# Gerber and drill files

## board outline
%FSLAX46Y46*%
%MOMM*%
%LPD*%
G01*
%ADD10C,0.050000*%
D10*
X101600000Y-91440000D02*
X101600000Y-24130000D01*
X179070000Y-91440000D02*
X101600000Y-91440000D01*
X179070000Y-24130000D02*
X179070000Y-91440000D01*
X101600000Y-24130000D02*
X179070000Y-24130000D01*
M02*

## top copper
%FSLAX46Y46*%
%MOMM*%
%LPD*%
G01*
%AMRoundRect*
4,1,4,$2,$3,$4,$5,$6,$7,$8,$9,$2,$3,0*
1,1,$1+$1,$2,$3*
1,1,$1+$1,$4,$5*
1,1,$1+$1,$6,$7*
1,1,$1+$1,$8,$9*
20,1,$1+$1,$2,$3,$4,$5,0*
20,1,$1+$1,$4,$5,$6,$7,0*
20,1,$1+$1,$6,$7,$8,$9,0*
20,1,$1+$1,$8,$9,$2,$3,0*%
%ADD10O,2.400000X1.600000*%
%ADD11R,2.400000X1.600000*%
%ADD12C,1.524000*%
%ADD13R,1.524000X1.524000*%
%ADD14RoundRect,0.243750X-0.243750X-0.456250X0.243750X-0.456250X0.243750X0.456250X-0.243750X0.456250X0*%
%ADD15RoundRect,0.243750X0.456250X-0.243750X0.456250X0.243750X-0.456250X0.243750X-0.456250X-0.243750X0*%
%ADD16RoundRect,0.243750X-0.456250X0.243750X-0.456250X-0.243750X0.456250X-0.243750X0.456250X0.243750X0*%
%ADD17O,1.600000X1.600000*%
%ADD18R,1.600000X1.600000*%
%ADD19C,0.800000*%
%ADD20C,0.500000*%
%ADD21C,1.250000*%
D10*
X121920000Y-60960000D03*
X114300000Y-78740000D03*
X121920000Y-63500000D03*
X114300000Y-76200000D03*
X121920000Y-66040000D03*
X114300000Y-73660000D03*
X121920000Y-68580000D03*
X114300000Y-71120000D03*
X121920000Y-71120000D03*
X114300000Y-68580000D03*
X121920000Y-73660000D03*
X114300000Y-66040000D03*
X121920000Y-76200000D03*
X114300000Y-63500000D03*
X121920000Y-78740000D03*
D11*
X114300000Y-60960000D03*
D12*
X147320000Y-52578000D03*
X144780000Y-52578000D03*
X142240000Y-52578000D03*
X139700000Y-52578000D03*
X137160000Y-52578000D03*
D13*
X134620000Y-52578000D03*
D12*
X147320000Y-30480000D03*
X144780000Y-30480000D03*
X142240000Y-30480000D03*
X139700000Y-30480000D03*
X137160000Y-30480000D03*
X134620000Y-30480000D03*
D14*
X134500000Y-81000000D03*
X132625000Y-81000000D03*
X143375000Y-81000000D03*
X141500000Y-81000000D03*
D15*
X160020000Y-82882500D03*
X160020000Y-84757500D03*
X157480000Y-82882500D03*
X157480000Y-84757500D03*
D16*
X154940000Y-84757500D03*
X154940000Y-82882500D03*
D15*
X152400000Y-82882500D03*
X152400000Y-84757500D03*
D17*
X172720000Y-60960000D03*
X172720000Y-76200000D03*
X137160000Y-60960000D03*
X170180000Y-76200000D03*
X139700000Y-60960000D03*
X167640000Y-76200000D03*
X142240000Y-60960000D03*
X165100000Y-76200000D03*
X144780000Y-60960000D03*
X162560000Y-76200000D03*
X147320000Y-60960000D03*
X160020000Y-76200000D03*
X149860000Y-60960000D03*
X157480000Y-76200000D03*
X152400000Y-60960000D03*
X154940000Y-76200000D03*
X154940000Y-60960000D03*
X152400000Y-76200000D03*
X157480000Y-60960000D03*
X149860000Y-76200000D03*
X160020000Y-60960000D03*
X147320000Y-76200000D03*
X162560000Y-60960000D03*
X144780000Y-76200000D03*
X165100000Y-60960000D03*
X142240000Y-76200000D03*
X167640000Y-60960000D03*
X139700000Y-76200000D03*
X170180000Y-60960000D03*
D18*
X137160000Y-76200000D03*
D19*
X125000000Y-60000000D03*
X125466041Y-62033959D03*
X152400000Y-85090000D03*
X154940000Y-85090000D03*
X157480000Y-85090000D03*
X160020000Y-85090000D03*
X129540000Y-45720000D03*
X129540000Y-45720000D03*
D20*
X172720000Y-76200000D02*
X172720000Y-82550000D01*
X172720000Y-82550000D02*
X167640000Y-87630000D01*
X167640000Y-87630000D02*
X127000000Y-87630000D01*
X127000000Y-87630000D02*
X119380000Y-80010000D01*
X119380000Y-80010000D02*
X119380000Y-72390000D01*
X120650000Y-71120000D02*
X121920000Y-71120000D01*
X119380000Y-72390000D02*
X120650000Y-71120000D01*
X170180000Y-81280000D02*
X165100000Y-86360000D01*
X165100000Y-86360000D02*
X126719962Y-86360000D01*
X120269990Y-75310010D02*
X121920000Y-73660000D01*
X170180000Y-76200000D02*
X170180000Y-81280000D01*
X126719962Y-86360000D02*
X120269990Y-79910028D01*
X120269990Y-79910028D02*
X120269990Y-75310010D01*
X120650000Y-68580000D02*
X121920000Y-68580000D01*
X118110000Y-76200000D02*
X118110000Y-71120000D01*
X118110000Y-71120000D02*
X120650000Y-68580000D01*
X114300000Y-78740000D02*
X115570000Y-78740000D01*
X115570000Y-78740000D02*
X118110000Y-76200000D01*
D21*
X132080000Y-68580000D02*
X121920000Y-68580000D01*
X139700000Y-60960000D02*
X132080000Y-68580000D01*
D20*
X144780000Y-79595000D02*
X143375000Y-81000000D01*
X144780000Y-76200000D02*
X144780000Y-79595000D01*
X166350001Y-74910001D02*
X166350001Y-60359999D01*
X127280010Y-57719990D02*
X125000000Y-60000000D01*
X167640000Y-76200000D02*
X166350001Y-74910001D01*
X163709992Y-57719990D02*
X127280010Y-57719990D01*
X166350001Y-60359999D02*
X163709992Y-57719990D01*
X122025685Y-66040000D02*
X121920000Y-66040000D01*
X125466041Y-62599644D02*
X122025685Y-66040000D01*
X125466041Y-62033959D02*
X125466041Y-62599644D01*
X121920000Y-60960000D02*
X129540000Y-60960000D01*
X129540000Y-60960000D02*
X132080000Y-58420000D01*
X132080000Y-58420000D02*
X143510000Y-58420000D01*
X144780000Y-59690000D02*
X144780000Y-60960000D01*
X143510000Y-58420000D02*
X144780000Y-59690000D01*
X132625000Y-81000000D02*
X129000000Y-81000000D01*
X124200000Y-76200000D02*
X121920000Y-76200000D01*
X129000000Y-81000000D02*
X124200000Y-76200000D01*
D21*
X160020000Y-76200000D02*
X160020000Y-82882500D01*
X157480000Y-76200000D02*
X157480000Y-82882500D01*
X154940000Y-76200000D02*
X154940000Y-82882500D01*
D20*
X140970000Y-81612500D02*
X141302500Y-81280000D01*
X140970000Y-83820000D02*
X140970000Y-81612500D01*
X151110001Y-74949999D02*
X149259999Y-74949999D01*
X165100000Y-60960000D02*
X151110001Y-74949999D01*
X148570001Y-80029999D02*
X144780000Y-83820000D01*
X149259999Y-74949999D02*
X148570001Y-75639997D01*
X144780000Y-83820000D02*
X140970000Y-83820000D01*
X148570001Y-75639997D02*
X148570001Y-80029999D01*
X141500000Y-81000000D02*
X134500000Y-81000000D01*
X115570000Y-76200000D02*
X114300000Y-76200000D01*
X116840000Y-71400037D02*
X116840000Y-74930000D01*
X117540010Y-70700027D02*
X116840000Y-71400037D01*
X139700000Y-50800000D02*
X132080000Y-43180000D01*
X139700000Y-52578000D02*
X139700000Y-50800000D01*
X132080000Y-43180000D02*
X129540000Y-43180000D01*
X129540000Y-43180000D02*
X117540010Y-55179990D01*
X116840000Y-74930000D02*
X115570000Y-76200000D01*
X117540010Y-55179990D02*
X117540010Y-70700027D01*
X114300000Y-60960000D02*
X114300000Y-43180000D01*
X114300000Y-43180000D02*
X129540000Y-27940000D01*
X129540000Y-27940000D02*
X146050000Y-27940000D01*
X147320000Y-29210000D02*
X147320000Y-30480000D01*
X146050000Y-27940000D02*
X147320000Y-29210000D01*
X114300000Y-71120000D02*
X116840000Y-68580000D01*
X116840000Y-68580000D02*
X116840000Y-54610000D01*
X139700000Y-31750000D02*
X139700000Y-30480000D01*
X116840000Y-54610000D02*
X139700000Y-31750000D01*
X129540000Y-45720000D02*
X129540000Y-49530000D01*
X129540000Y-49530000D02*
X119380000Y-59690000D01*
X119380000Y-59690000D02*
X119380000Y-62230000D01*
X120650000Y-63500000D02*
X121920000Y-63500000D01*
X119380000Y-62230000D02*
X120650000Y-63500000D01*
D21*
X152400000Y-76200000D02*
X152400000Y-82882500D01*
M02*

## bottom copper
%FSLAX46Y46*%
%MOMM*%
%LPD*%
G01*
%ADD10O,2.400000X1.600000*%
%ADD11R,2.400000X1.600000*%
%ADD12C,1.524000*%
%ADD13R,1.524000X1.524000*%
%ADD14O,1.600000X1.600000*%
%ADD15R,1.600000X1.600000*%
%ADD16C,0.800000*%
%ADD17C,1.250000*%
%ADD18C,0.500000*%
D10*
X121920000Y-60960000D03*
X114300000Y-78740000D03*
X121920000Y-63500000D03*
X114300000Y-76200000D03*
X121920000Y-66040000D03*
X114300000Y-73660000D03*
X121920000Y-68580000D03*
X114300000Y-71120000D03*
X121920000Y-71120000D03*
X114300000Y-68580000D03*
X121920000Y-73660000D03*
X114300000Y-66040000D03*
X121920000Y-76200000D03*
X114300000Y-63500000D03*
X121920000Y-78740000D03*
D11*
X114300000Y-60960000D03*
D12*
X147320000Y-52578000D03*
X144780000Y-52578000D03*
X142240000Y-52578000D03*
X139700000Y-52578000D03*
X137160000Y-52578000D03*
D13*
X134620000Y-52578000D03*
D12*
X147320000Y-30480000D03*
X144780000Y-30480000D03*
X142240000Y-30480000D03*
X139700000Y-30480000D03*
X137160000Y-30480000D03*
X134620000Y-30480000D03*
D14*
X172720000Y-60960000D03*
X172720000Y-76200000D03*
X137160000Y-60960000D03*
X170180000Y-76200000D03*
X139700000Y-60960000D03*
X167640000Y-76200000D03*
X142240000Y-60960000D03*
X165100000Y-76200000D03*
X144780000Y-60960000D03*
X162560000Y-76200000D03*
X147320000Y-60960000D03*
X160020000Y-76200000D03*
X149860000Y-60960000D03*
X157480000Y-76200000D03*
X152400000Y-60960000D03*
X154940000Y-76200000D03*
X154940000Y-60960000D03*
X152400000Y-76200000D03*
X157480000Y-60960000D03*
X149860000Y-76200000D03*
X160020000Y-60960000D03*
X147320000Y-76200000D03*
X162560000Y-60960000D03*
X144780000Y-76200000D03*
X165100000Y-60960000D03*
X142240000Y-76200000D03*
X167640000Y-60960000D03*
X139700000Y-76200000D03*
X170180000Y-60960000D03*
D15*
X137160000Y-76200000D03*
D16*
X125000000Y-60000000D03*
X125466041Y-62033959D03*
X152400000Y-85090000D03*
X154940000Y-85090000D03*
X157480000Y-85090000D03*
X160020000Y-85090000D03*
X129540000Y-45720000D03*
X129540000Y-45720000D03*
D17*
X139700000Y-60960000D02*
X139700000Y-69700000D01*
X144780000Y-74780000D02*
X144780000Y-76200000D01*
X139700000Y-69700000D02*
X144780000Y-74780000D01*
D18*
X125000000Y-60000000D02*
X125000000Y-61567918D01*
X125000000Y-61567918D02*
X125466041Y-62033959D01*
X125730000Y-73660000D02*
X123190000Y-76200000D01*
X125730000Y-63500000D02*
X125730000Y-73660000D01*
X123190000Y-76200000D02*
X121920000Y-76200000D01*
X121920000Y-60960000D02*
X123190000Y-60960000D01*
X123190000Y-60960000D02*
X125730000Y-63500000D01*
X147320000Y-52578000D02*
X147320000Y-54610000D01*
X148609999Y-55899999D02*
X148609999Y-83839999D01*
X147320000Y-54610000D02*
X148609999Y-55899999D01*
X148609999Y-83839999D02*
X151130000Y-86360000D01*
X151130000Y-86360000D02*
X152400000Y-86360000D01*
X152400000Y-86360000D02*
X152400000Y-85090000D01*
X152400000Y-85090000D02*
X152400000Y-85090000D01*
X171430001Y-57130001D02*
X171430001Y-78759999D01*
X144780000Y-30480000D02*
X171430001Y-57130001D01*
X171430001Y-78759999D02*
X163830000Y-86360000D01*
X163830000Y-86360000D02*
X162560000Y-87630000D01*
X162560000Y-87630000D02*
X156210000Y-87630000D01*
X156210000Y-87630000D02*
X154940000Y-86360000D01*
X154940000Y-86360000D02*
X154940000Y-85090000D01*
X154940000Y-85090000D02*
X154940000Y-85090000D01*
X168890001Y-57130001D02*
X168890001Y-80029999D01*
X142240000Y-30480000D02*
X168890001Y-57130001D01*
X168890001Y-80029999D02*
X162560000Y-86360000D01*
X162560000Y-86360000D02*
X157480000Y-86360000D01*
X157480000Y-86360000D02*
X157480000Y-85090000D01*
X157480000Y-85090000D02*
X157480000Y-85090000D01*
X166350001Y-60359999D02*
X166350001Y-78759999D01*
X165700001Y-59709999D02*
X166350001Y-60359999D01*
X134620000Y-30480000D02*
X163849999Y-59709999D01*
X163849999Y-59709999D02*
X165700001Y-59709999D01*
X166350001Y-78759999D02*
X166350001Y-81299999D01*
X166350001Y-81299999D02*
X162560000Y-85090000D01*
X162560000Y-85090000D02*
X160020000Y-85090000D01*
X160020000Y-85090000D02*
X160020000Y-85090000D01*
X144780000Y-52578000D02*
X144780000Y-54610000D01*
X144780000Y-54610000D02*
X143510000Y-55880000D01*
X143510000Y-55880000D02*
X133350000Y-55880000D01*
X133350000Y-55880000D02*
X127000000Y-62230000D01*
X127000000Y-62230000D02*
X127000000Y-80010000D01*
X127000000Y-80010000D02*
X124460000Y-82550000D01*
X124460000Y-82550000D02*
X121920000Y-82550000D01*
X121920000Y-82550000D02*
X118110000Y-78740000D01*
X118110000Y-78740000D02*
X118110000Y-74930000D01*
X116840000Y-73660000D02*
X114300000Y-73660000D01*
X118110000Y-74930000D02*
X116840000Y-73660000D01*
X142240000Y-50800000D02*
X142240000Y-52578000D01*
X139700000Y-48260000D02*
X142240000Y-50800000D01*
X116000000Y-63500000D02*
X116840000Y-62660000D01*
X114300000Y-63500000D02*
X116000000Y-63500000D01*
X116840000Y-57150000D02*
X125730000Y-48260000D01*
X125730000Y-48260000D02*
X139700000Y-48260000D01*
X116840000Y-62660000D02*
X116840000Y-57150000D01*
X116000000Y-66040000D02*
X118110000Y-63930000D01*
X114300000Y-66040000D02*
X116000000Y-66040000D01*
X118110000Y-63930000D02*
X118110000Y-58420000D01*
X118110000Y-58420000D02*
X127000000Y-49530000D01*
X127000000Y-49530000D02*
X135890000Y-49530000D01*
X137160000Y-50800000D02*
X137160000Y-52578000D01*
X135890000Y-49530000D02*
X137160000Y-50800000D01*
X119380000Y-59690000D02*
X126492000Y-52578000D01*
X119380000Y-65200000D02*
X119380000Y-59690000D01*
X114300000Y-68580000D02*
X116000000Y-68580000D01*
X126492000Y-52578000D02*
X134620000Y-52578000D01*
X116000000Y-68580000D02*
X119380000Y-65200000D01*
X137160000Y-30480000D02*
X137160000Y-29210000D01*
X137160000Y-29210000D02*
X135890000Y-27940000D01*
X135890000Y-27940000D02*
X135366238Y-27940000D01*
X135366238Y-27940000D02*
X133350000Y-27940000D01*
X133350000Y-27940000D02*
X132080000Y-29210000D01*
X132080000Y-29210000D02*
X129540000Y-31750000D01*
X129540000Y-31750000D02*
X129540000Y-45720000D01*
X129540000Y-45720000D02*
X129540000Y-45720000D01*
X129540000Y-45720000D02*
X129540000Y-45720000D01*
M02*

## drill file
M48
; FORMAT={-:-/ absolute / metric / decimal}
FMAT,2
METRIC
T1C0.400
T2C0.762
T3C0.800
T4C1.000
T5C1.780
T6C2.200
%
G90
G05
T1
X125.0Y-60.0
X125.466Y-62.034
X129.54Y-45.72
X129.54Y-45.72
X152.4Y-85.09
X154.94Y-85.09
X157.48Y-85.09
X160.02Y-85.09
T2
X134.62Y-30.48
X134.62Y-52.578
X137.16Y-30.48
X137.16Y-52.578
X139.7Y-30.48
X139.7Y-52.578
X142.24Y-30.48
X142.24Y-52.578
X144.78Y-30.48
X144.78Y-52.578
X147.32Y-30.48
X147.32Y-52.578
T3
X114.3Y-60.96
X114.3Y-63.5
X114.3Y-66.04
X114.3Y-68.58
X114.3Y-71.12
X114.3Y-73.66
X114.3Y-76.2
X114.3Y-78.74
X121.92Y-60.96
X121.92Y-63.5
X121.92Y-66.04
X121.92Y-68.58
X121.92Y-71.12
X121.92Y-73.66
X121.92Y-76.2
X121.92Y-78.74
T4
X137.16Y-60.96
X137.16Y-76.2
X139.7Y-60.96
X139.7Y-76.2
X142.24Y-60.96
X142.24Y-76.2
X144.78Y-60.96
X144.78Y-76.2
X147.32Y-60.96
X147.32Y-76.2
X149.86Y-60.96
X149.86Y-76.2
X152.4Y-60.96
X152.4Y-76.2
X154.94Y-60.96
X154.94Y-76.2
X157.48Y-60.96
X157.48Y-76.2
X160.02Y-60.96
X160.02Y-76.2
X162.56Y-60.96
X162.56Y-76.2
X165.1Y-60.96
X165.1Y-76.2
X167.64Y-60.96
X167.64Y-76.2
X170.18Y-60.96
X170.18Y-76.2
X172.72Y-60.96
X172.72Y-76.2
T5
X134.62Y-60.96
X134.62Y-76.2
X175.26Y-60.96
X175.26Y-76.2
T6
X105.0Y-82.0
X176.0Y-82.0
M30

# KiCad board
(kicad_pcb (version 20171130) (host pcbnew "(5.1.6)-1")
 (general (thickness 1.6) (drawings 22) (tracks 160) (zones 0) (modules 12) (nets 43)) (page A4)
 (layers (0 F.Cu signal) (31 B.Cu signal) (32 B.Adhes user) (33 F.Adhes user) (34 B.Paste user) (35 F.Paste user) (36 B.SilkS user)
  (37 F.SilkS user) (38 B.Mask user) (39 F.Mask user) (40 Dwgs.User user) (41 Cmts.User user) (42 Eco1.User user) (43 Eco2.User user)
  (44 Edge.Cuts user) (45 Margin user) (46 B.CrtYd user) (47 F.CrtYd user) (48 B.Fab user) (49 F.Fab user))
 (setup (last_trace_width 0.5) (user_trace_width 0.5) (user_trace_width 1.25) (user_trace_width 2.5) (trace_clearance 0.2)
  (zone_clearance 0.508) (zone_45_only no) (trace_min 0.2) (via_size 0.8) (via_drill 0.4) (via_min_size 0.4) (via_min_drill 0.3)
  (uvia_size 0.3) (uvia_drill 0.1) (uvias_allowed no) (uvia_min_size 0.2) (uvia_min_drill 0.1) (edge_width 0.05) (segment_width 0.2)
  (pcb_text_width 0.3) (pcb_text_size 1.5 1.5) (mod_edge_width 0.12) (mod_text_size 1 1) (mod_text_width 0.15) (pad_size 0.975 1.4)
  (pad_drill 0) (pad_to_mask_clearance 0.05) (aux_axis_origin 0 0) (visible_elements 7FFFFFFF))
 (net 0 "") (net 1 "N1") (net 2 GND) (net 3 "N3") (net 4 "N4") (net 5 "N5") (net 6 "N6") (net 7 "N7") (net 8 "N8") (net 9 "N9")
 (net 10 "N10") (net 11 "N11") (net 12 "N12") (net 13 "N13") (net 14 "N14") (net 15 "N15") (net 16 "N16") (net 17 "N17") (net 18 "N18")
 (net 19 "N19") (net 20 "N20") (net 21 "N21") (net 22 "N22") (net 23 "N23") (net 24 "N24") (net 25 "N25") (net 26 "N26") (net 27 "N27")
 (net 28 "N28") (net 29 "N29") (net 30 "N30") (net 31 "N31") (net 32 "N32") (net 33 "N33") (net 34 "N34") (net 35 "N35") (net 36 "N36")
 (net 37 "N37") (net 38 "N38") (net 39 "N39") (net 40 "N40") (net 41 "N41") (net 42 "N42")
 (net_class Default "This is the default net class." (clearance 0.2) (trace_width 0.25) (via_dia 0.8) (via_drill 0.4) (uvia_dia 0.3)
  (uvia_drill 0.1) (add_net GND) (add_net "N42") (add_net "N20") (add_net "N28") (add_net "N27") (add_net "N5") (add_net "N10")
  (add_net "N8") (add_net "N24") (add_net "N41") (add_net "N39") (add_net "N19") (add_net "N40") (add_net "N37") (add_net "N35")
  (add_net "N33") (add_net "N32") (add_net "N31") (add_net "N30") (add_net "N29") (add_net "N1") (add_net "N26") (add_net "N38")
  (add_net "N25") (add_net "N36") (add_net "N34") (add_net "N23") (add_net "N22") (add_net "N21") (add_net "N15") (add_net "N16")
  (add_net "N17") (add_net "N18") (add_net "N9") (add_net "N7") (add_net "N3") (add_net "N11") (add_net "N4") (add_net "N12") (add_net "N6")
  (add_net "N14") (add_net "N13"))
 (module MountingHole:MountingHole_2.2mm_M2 (layer F.Cu) (at 176 82)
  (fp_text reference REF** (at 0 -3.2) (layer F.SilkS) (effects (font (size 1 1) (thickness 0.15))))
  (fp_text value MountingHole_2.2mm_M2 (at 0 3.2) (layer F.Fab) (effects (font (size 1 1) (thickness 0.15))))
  (pad 1 np_thru_hole circle (at 0 0) (size 2.2 2.2) (drill 2.2) (layers *.Cu *.Mask)))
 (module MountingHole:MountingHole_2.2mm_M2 (layer F.Cu) (at 105 82)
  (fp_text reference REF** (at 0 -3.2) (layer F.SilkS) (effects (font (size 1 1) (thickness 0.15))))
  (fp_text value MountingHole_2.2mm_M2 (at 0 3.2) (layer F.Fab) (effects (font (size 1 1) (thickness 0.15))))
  (pad 1 np_thru_hole circle (at 0 0) (size 2.2 2.2) (drill 2.2) (layers *.Cu *.Mask)))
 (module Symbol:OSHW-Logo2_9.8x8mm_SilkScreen (layer F.Cu) (at 128.27 86.36)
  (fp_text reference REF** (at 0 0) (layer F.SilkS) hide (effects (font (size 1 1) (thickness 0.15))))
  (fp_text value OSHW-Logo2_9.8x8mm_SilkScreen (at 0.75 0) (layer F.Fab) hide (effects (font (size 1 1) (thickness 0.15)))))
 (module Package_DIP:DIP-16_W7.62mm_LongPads (layer F.Cu) (at 114.3 60.96)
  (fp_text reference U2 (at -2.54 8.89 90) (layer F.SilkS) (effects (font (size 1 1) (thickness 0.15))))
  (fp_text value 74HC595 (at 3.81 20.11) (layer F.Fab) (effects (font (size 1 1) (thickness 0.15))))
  (pad 16 thru_hole oval (at 7.62 0) (size 2.4 1.6) (drill 0.8) (layers *.Cu *.Mask) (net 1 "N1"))
  (pad 8 thru_hole oval (at 0 17.78) (size 2.4 1.6) (drill 0.8) (layers *.Cu *.Mask) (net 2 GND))
  (pad 15 thru_hole oval (at 7.62 2.54) (size 2.4 1.6) (drill 0.8) (layers *.Cu *.Mask) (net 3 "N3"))
  (pad 7 thru_hole oval (at 0 15.24) (size 2.4 1.6) (drill 0.8) (layers *.Cu *.Mask) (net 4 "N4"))
  (pad 14 thru_hole oval (at 7.62 5.08) (size 2.4 1.6) (drill 0.8) (layers *.Cu *.Mask) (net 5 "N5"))
  (pad 6 thru_hole oval (at 0 12.7) (size 2.4 1.6) (drill 0.8) (layers *.Cu *.Mask) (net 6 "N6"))
  (pad 13 thru_hole oval (at 7.62 7.62) (size 2.4 1.6) (drill 0.8) (layers *.Cu *.Mask) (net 2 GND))
  (pad 5 thru_hole oval (at 0 10.16) (size 2.4 1.6) (drill 0.8) (layers *.Cu *.Mask) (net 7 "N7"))
  (pad 12 thru_hole oval (at 7.62 10.16) (size 2.4 1.6) (drill 0.8) (layers *.Cu *.Mask) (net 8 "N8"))
  (pad 4 thru_hole oval (at 0 7.62) (size 2.4 1.6) (drill 0.8) (layers *.Cu *.Mask) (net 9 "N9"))
  (pad 11 thru_hole oval (at 7.62 12.7) (size 2.4 1.6) (drill 0.8) (layers *.Cu *.Mask) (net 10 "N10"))
  (pad 3 thru_hole oval (at 0 5.08) (size 2.4 1.6) (drill 0.8) (layers *.Cu *.Mask) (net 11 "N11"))
  (pad 10 thru_hole oval (at 7.62 15.24) (size 2.4 1.6) (drill 0.8) (layers *.Cu *.Mask) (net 1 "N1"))
  (pad 2 thru_hole oval (at 0 2.54) (size 2.4 1.6) (drill 0.8) (layers *.Cu *.Mask) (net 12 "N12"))
  (pad 9 thru_hole oval (at 7.62 17.78) (size 2.4 1.6) (drill 0.8) (layers *.Cu *.Mask) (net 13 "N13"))
  (pad 1 thru_hole rect (at 0 0) (size 2.4 1.6) (drill 0.8) (layers *.Cu *.Mask) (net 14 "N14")))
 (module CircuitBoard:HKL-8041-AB (layer F.Cu) (at 139.7 27.94)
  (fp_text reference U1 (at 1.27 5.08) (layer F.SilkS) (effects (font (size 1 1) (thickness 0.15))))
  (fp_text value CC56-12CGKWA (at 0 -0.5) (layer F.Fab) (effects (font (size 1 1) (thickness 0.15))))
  (pad 6 thru_hole circle (at 7.62 24.638) (size 1.524 1.524) (drill 0.762) (layers *.Cu *.Mask) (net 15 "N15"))
  (pad 5 thru_hole circle (at 5.08 24.638) (size 1.524 1.524) (drill 0.762) (layers *.Cu *.Mask) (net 6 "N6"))
  (pad 4 thru_hole circle (at 2.54 24.638) (size 1.524 1.524) (drill 0.762) (layers *.Cu *.Mask) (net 12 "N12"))
  (pad 3 thru_hole circle (at 0 24.638) (size 1.524 1.524) (drill 0.762) (layers *.Cu *.Mask) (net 4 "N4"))
  (pad 2 thru_hole circle (at -2.54 24.638) (size 1.524 1.524) (drill 0.762) (layers *.Cu *.Mask) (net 11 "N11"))
  (pad 1 thru_hole rect (at -5.08 24.638) (size 1.524 1.524) (drill 0.762) (layers *.Cu *.Mask) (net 9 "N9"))
  (pad 7 thru_hole circle (at 7.62 2.54) (size 1.524 1.524) (drill 0.762) (layers *.Cu *.Mask) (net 14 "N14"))
  (pad 8 thru_hole circle (at 5.08 2.54) (size 1.524 1.524) (drill 0.762) (layers *.Cu *.Mask) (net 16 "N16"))
  (pad 9 thru_hole circle (at 2.54 2.54) (size 1.524 1.524) (drill 0.762) (layers *.Cu *.Mask) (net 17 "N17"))
  (pad 10 thru_hole circle (at 0 2.54) (size 1.524 1.524) (drill 0.762) (layers *.Cu *.Mask) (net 7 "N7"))
  (pad 11 thru_hole circle (at -2.54 2.54) (size 1.524 1.524) (drill 0.762) (layers *.Cu *.Mask) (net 3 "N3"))
  (pad 12 thru_hole circle (at -5.08 2.54) (size 1.524 1.524) (drill 0.762) (layers *.Cu *.Mask) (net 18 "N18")))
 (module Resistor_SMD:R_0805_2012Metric (layer F.Cu) (at 133.5625 81)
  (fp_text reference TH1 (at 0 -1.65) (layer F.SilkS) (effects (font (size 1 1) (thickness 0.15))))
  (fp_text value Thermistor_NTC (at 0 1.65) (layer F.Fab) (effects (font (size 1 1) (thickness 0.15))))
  (pad 2 smd roundrect (at 0.9375 0) (size 0.975 1.4) (layers F.Cu F.Paste F.Mask) (roundrect_rratio 0.25) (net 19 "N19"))
  (pad 1 smd roundrect (at -0.9375 0) (size 0.975 1.4) (layers F.Cu F.Paste F.Mask) (roundrect_rratio 0.25) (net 1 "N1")))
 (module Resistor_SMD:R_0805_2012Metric (layer F.Cu) (at 142.4375 81)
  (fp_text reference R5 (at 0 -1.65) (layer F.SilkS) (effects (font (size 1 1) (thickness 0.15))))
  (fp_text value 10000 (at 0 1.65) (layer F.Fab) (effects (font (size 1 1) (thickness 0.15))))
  (pad 2 smd roundrect (at 0.9375 0) (size 0.975 1.4) (layers F.Cu F.Paste F.Mask) (roundrect_rratio 0.25) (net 2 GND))
  (pad 1 smd roundrect (at -0.9375 0) (size 0.975 1.4) (layers F.Cu F.Paste F.Mask) (roundrect_rratio 0.25) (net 19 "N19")))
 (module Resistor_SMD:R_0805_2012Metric (layer F.Cu) (at 160.02 83.82 90)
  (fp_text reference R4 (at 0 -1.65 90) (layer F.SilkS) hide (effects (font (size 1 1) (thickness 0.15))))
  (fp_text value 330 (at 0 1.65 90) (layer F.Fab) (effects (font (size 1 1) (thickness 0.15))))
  (pad 2 smd roundrect (at 0.9375 0 90) (size 0.975 1.4) (layers F.Cu F.Paste F.Mask) (roundrect_rratio 0.25) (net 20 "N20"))
  (pad 1 smd roundrect (at -0.9375 0 90) (size 0.975 1.4) (layers F.Cu F.Paste F.Mask) (roundrect_rratio 0.25) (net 18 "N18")))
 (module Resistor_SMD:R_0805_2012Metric (layer F.Cu) (at 157.48 83.82 90)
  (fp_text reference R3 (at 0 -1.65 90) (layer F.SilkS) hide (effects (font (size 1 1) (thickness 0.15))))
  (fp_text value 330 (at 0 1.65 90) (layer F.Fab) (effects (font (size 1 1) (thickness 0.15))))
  (pad 2 smd roundrect (at 0.9375 0 90) (size 0.975 1.4) (layers F.Cu F.Paste F.Mask) (roundrect_rratio 0.25) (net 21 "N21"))
  (pad 1 smd roundrect (at -0.9375 0 90) (size 0.975 1.4) (layers F.Cu F.Paste F.Mask) (roundrect_rratio 0.25) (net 17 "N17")))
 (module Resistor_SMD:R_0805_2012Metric (layer F.Cu) (at 154.94 83.82 270)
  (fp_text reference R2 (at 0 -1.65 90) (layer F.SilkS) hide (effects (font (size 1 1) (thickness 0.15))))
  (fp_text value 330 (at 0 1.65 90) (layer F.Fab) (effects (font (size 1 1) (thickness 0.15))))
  (pad 2 smd roundrect (at 0.9375 0 270) (size 0.975 1.4) (layers F.Cu F.Paste F.Mask) (roundrect_rratio 0.25) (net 16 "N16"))
  (pad 1 smd roundrect (at -0.9375 0 270) (size 0.975 1.4) (layers F.Cu F.Paste F.Mask) (roundrect_rratio 0.25) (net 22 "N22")))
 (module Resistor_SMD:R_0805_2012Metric (layer F.Cu) (at 152.4 83.82 90)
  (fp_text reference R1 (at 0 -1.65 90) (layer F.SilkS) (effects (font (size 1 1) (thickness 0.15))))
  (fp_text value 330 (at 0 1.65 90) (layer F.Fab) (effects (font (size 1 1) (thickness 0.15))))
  (pad 2 smd roundrect (at 0.9375 0 90) (size 0.975 1.4) (layers F.Cu F.Paste F.Mask) (roundrect_rratio 0.25) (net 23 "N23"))
  (pad 1 smd roundrect (at -0.9375 0 90) (size 0.975 1.4) (layers F.Cu F.Paste F.Mask) (roundrect_rratio 0.25) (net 15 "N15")))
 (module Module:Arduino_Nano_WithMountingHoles (layer F.Cu) (at 137.16 76.2 90)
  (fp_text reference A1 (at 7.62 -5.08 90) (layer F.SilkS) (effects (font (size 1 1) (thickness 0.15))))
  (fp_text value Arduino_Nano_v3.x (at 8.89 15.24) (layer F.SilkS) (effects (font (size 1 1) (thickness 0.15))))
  (pad "" np_thru_hole circle (at 0 38.1 90) (size 1.78 1.78) (drill 1.78) (layers *.Cu *.Mask))
  (pad "" np_thru_hole circle (at 15.24 38.1 90) (size 1.78 1.78) (drill 1.78) (layers *.Cu *.Mask))
  (pad "" np_thru_hole circle (at 15.24 -2.54 90) (size 1.78 1.78) (drill 1.78) (layers *.Cu *.Mask))
  (pad "" np_thru_hole circle (at 0 -2.54 90) (size 1.78 1.78) (drill 1.78) (layers *.Cu *.Mask))
  (pad 16 thru_hole oval (at 15.24 35.56 90) (size 1.6 1.6) (drill 1) (layers *.Cu *.Mask) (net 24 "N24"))
  (pad 15 thru_hole oval (at 0 35.56 90) (size 1.6 1.6) (drill 1) (layers *.Cu *.Mask) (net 8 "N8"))
  (pad 30 thru_hole oval (at 15.24 0 90) (size 1.6 1.6) (drill 1) (layers *.Cu *.Mask) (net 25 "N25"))
  (pad 14 thru_hole oval (at 0 33.02 90) (size 1.6 1.6) (drill 1) (layers *.Cu *.Mask) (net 10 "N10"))
  (pad 29 thru_hole oval (at 15.24 2.54 90) (size 1.6 1.6) (drill 1) (layers *.Cu *.Mask) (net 2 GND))
  (pad 13 thru_hole oval (at 0 30.48 90) (size 1.6 1.6) (drill 1) (layers *.Cu *.Mask) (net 5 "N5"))
  (pad 28 thru_hole oval (at 15.24 5.08 90) (size 1.6 1.6) (drill 1) (layers *.Cu *.Mask) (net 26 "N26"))
  (pad 12 thru_hole oval (at 0 27.94 90) (size 1.6 1.6) (drill 1) (layers *.Cu *.Mask) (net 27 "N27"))
  (pad 27 thru_hole oval (at 15.24 7.62 90) (size 1.6 1.6) (drill 1) (layers *.Cu *.Mask) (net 1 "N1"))
  (pad 11 thru_hole oval (at 0 25.4 90) (size 1.6 1.6) (drill 1) (layers *.Cu *.Mask) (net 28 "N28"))
  (pad 26 thru_hole oval (at 15.24 10.16 90) (size 1.6 1.6) (drill 1) (layers *.Cu *.Mask) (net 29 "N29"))
  (pad 10 thru_hole oval (at 0 22.86 90) (size 1.6 1.6) (drill 1) (layers *.Cu *.Mask) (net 20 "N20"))
  (pad 25 thru_hole oval (at 15.24 12.7 90) (size 1.6 1.6) (drill 1) (layers *.Cu *.Mask) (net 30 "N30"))
  (pad 9 thru_hole oval (at 0 20.32 90) (size 1.6 1.6) (drill 1) (layers *.Cu *.Mask) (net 21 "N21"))
  (pad 24 thru_hole oval (at 15.24 15.24 90) (size 1.6 1.6) (drill 1) (layers *.Cu *.Mask) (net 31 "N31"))
  (pad 8 thru_hole oval (at 0 17.78 90) (size 1.6 1.6) (drill 1) (layers *.Cu *.Mask) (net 22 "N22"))
  (pad 23 thru_hole oval (at 15.24 17.78 90) (size 1.6 1.6) (drill 1) (layers *.Cu *.Mask) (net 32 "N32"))
  (pad 7 thru_hole oval (at 0 15.24 90) (size 1.6 1.6) (drill 1) (layers *.Cu *.Mask) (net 23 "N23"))
  (pad 22 thru_hole oval (at 15.24 20.32 90) (size 1.6 1.6) (drill 1) (layers *.Cu *.Mask) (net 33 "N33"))
  (pad 6 thru_hole oval (at 0 12.7 90) (size 1.6 1.6) (drill 1) (layers *.Cu *.Mask) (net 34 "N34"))
  (pad 21 thru_hole oval (at 15.24 22.86 90) (size 1.6 1.6) (drill 1) (layers *.Cu *.Mask) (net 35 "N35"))
  (pad 5 thru_hole oval (at 0 10.16 90) (size 1.6 1.6) (drill 1) (layers *.Cu *.Mask) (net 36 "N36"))
  (pad 20 thru_hole oval (at 15.24 25.4 90) (size 1.6 1.6) (drill 1) (layers *.Cu *.Mask) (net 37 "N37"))
  (pad 4 thru_hole oval (at 0 7.62 90) (size 1.6 1.6) (drill 1) (layers *.Cu *.Mask) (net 2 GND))
  (pad 19 thru_hole oval (at 15.24 27.94 90) (size 1.6 1.6) (drill 1) (layers *.Cu *.Mask) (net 19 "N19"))
  (pad 3 thru_hole oval (at 0 5.08 90) (size 1.6 1.6) (drill 1) (layers *.Cu *.Mask) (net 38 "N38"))
  (pad 18 thru_hole oval (at 15.24 30.48 90) (size 1.6 1.6) (drill 1) (layers *.Cu *.Mask) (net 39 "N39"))
  (pad 2 thru_hole oval (at 0 2.54 90) (size 1.6 1.6) (drill 1) (layers *.Cu *.Mask) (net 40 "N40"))
  (pad 17 thru_hole oval (at 15.24 33.02 90) (size 1.6 1.6) (drill 1) (layers *.Cu *.Mask) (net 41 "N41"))
  (pad 1 thru_hole rect (at 0 0 90) (size 1.6 1.6) (drill 1) (layers *.Cu *.Mask) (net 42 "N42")))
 (gr_line (start 101.6 91.44) (end 101.6 24.13) (layer Edge.Cuts) (width 0.05))
 (gr_line (start 179.07 91.44) (end 101.6 91.44) (layer Edge.Cuts) (width 0.05))
 (gr_line (start 179.07 24.13) (end 179.07 91.44) (layer Edge.Cuts) (width 0.05))
 (gr_line (start 101.6 24.13) (end 179.07 24.13) (layer Edge.Cuts) (width 0.05))
 (segment (start 172.72 76.2) (end 172.72 82.55) (width 0.5) (layer F.Cu) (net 8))
 (segment (start 172.72 82.55) (end 167.64 87.63) (width 0.5) (layer F.Cu) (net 8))
 (segment (start 167.64 87.63) (end 127 87.63) (width 0.5) (layer F.Cu) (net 8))
 (segment (start 127 87.63) (end 119.38 80.01) (width 0.5) (layer F.Cu) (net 8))
 (segment (start 119.38 80.01) (end 119.38 72.39) (width 0.5) (layer F.Cu) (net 8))
 (segment (start 120.65 71.12) (end 121.92 71.12) (width 0.5) (layer F.Cu) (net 8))
 (segment (start 119.38 72.39) (end 120.65 71.12) (width 0.5) (layer F.Cu) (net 8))
 (segment (start 170.18 81.28) (end 165.1 86.36) (width 0.5) (layer F.Cu) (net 10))
 (segment (start 165.1 86.36) (end 126.719962 86.36) (width 0.5) (layer F.Cu) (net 10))
 (segment (start 120.26999 75.31001) (end 121.92 73.66) (width 0.5) (layer F.Cu) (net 10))
 (segment (start 170.18 76.2) (end 170.18 81.28) (width 0.5) (layer F.Cu) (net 10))
 (segment (start 126.719962 86.36) (end 120.26999 79.910028) (width 0.5) (layer F.Cu) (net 10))
 (segment (start 120.26999 79.910028) (end 120.26999 75.31001) (width 0.5) (layer F.Cu) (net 10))
 (segment (start 120.65 68.58) (end 121.92 68.58) (width 0.5) (layer F.Cu) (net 2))
 (segment (start 118.11 76.2) (end 118.11 71.12) (width 0.5) (layer F.Cu) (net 2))
 (segment (start 118.11 71.12) (end 120.65 68.58) (width 0.5) (layer F.Cu) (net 2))
 (segment (start 114.3 78.74) (end 115.57 78.74) (width 0.5) (layer F.Cu) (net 2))
 (segment (start 115.57 78.74) (end 118.11 76.2) (width 0.5) (layer F.Cu) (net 2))
 (segment (start 132.08 68.58) (end 121.92 68.58) (width 1.25) (layer F.Cu) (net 2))
 (segment (start 139.7 60.96) (end 132.08 68.58) (width 1.25) (layer F.Cu) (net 2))
 (segment (start 139.7 60.96) (end 139.7 69.7) (width 1.25) (layer B.Cu) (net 2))
 (segment (start 144.78 74.78) (end 144.78 76.2) (width 1.25) (layer B.Cu) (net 2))
 (segment (start 139.7 69.7) (end 144.78 74.78) (width 1.25) (layer B.Cu) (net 2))
 (segment (start 144.78 79.595) (end 143.375 81) (width 0.5) (layer F.Cu) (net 2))
 (segment (start 144.78 76.2) (end 144.78 79.595) (width 0.5) (layer F.Cu) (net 2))
 (segment (start 166.350001 74.910001) (end 166.350001 60.359999) (width 0.5) (layer F.Cu) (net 5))
 (segment (start 127.28001 57.71999) (end 125 60) (width 0.5) (layer F.Cu) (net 5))
 (segment (start 167.64 76.2) (end 166.350001 74.910001) (width 0.5) (layer F.Cu) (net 5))
 (segment (start 163.709992 57.71999) (end 127.28001 57.71999) (width 0.5) (layer F.Cu) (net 5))
 (via (at 125 60) (size 0.8) (drill 0.4) (layers F.Cu B.Cu) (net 5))
 (segment (start 166.350001 60.359999) (end 163.709992 57.71999) (width 0.5) (layer F.Cu) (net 5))
 (via (at 125.466041 62.033959) (size 0.8) (drill 0.4) (layers F.Cu B.Cu) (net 5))
 (segment (start 125 60) (end 125 61.567918) (width 0.5) (layer B.Cu) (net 5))
 (segment (start 125 61.567918) (end 125.466041 62.033959) (width 0.5) (layer B.Cu) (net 5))
 (segment (start 122.025685 66.04) (end 121.92 66.04) (width 0.5) (layer F.Cu) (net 5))
 (segment (start 125.466041 62.599644) (end 122.025685 66.04) (width 0.5) (layer F.Cu) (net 5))
 (segment (start 125.466041 62.033959) (end 125.466041 62.599644) (width 0.5) (layer F.Cu) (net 5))
 (segment (start 121.92 60.96) (end 129.54 60.96) (width 0.5) (layer F.Cu) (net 1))
 (segment (start 129.54 60.96) (end 132.08 58.42) (width 0.5) (layer F.Cu) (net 1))
 (segment (start 132.08 58.42) (end 143.51 58.42) (width 0.5) (layer F.Cu) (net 1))
 (segment (start 144.78 59.69) (end 144.78 60.96) (width 0.5) (layer F.Cu) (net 1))
 (segment (start 143.51 58.42) (end 144.78 59.69) (width 0.5) (layer F.Cu) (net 1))
 (segment (start 125.73 73.66) (end 123.19 76.2) (width 0.5) (layer B.Cu) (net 1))
 (segment (start 125.73 63.5) (end 125.73 73.66) (width 0.5) (layer B.Cu) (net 1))
 (segment (start 123.19 76.2) (end 121.92 76.2) (width 0.5) (layer B.Cu) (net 1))
 (segment (start 121.92 60.96) (end 123.19 60.96) (width 0.5) (layer B.Cu) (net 1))
 (segment (start 123.19 60.96) (end 125.73 63.5) (width 0.5) (layer B.Cu) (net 1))
 (segment (start 132.625 81) (end 129 81) (width 0.5) (layer F.Cu) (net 1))
 (segment (start 124.2 76.2) (end 121.92 76.2) (width 0.5) (layer F.Cu) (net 1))
 (segment (start 129 81) (end 124.2 76.2) (width 0.5) (layer F.Cu) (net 1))
 (segment (start 160.02 76.2) (end 160.02 82.8825) (width 1.25) (layer F.Cu) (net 20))
 (segment (start 157.48 76.2) (end 157.48 82.8825) (width 1.25) (layer F.Cu) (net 21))
 (segment (start 154.94 76.2) (end 154.94 82.8825) (width 1.25) (layer F.Cu) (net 22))
 (segment (start 140.97 81.6125) (end 141.3025 81.28) (width 0.5) (layer F.Cu) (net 19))
 (segment (start 140.97 83.82) (end 140.97 81.6125) (width 0.5) (layer F.Cu) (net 19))
 (segment (start 151.110001 74.949999) (end 149.259999 74.949999) (width 0.5) (layer F.Cu) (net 19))
 (segment (start 165.1 60.96) (end 151.110001 74.949999) (width 0.5) (layer F.Cu) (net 19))
 (segment (start 148.570001 80.029999) (end 144.78 83.82) (width 0.5) (layer F.Cu) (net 19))
 (segment (start 149.259999 74.949999) (end 148.570001 75.639997) (width 0.5) (layer F.Cu) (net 19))
 (segment (start 144.78 83.82) (end 140.97 83.82) (width 0.5) (layer F.Cu) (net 19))
 (segment (start 148.570001 75.639997) (end 148.570001 80.029999) (width 0.5) (layer F.Cu) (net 19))
 (segment (start 141.5 81) (end 134.5 81) (width 0.5) (layer F.Cu) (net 19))
 (segment (start 147.32 52.578) (end 147.32 54.61) (width 0.5) (layer B.Cu) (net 15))
 (segment (start 148.609999 55.899999) (end 148.609999 83.839999) (width 0.5) (layer B.Cu) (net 15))
 (segment (start 147.32 54.61) (end 148.609999 55.899999) (width 0.5) (layer B.Cu) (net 15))
 (segment (start 148.609999 83.839999) (end 151.13 86.36) (width 0.5) (layer B.Cu) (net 15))
 (segment (start 151.13 86.36) (end 152.4 86.36) (width 0.5) (layer B.Cu) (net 15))
 (segment (start 152.4 86.36) (end 152.4 85.09) (width 0.5) (layer B.Cu) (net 15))
 (segment (start 152.4 85.09) (end 152.4 85.09) (width 0.5) (layer B.Cu) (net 15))
 (via (at 152.4 85.09) (size 0.8) (drill 0.4) (layers F.Cu B.Cu) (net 15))
 (segment (start 171.430001 57.130001) (end 171.430001 78.759999) (width 0.5) (layer B.Cu) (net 16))
 (segment (start 144.78 30.48) (end 171.430001 57.130001) (width 0.5) (layer B.Cu) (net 16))
 (segment (start 171.430001 78.759999) (end 163.83 86.36) (width 0.5) (layer B.Cu) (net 16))
 (segment (start 163.83 86.36) (end 162.56 87.63) (width 0.5) (layer B.Cu) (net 16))
 (segment (start 162.56 87.63) (end 156.21 87.63) (width 0.5) (layer B.Cu) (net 16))
 (segment (start 156.21 87.63) (end 154.94 86.36) (width 0.5) (layer B.Cu) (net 16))
 (segment (start 154.94 86.36) (end 154.94 85.09) (width 0.5) (layer B.Cu) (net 16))
 (segment (start 154.94 85.09) (end 154.94 85.09) (width 0.5) (layer B.Cu) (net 16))
 (via (at 154.94 85.09) (size 0.8) (drill 0.4) (layers F.Cu B.Cu) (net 16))
 (segment (start 168.890001 57.130001) (end 168.890001 80.029999) (width 0.5) (layer B.Cu) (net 17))
 (segment (start 142.24 30.48) (end 168.890001 57.130001) (width 0.5) (layer B.Cu) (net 17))
 (segment (start 168.890001 80.029999) (end 162.56 86.36) (width 0.5) (layer B.Cu) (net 17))
 (segment (start 162.56 86.36) (end 157.48 86.36) (width 0.5) (layer B.Cu) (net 17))
 (segment (start 157.48 86.36) (end 157.48 85.09) (width 0.5) (layer B.Cu) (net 17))
 (segment (start 157.48 85.09) (end 157.48 85.09) (width 0.5) (layer B.Cu) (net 17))
 (via (at 157.48 85.09) (size 0.8) (drill 0.4) (layers F.Cu B.Cu) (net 17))
 (segment (start 166.350001 60.359999) (end 166.350001 78.759999) (width 0.5) (layer B.Cu) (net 18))
 (segment (start 165.700001 59.709999) (end 166.350001 60.359999) (width 0.5) (layer B.Cu) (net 18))
 (segment (start 134.62 30.48) (end 163.849999 59.709999) (width 0.5) (layer B.Cu) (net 18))
 (segment (start 163.849999 59.709999) (end 165.700001 59.709999) (width 0.5) (layer B.Cu) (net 18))
 (segment (start 166.350001 78.759999) (end 166.350001 81.299999) (width 0.5) (layer B.Cu) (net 18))
 (segment (start 166.350001 81.299999) (end 162.56 85.09) (width 0.5) (layer B.Cu) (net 18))
 (segment (start 162.56 85.09) (end 160.02 85.09) (width 0.5) (layer B.Cu) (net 18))
 (segment (start 160.02 85.09) (end 160.02 85.09) (width 0.5) (layer B.Cu) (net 18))
 (via (at 160.02 85.09) (size 0.8) (drill 0.4) (layers F.Cu B.Cu) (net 18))
 (segment (start 144.78 52.578) (end 144.78 54.61) (width 0.5) (layer B.Cu) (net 6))
 (segment (start 144.78 54.61) (end 143.51 55.88) (width 0.5) (layer B.Cu) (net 6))
 (segment (start 143.51 55.88) (end 133.35 55.88) (width 0.5) (layer B.Cu) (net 6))
 (segment (start 133.35 55.88) (end 127 62.23) (width 0.5) (layer B.Cu) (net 6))
 (segment (start 127 62.23) (end 127 80.01) (width 0.5) (layer B.Cu) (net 6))
 (segment (start 127 80.01) (end 124.46 82.55) (width 0.5) (layer B.Cu) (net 6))
 (segment (start 124.46 82.55) (end 121.92 82.55) (width 0.5) (layer B.Cu) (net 6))
 (segment (start 121.92 82.55) (end 118.11 78.74) (width 0.5) (layer B.Cu) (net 6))
 (segment (start 118.11 78.74) (end 118.11 74.93) (width 0.5) (layer B.Cu) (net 6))
 (segment (start 116.84 73.66) (end 114.3 73.66) (width 0.5) (layer B.Cu) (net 6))
 (segment (start 118.11 74.93) (end 116.84 73.66) (width 0.5) (layer B.Cu) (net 6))
 (segment (start 142.24 50.8) (end 142.24 52.578) (width 0.5) (layer B.Cu) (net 12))
 (segment (start 139.7 48.26) (end 142.24 50.8) (width 0.5) (layer B.Cu) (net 12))
 (segment (start 116 63.5) (end 116.84 62.66) (width 0.5) (layer B.Cu) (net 12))
 (segment (start 114.3 63.5) (end 116 63.5) (width 0.5) (layer B.Cu) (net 12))
 (segment (start 116.84 57.15) (end 125.73 48.26) (width 0.5) (layer B.Cu) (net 12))
 (segment (start 125.73 48.26) (end 139.7 48.26) (width 0.5) (layer B.Cu) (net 12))
 (segment (start 116.84 62.66) (end 116.84 57.15) (width 0.5) (layer B.Cu) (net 12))
 (segment (start 115.57 76.2) (end 114.3 76.2) (width 0.5) (layer F.Cu) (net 4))
 (segment (start 116.84 71.400037) (end 116.84 74.93) (width 0.5) (layer F.Cu) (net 4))
 (segment (start 117.54001 70.700027) (end 116.84 71.400037) (width 0.5) (layer F.Cu) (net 4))
 (segment (start 139.7 50.8) (end 132.08 43.18) (width 0.5) (layer F.Cu) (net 4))
 (segment (start 139.7 52.578) (end 139.7 50.8) (width 0.5) (layer F.Cu) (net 4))
 (segment (start 132.08 43.18) (end 129.54 43.18) (width 0.5) (layer F.Cu) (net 4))
 (segment (start 129.54 43.18) (end 117.54001 55.17999) (width 0.5) (layer F.Cu) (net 4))
 (segment (start 116.84 74.93) (end 115.57 76.2) (width 0.5) (layer F.Cu) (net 4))
 (segment (start 117.54001 55.17999) (end 117.54001 70.700027) (width 0.5) (layer F.Cu) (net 4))
 (segment (start 116 66.04) (end 118.11 63.93) (width 0.5) (layer B.Cu) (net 11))
 (segment (start 114.3 66.04) (end 116 66.04) (width 0.5) (layer B.Cu) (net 11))
 (segment (start 118.11 63.93) (end 118.11 58.42) (width 0.5) (layer B.Cu) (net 11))
 (segment (start 118.11 58.42) (end 127 49.53) (width 0.5) (layer B.Cu) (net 11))
 (segment (start 127 49.53) (end 135.89 49.53) (width 0.5) (layer B.Cu) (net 11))
 (segment (start 137.16 50.8) (end 137.16 52.578) (width 0.5) (layer B.Cu) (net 11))
 (segment (start 135.89 49.53) (end 137.16 50.8) (width 0.5) (layer B.Cu) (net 11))
 (segment (start 119.38 59.69) (end 126.492 52.578) (width 0.5) (layer B.Cu) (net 9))
 (segment (start 119.38 65.2) (end 119.38 59.69) (width 0.5) (layer B.Cu) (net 9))
 (segment (start 114.3 68.58) (end 116 68.58) (width 0.5) (layer B.Cu) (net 9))
 (segment (start 126.492 52.578) (end 134.62 52.578) (width 0.5) (layer B.Cu) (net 9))
 (segment (start 116 68.58) (end 119.38 65.2) (width 0.5) (layer B.Cu) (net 9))
 (segment (start 114.3 60.96) (end 114.3 43.18) (width 0.5) (layer F.Cu) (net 14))
 (segment (start 114.3 43.18) (end 129.54 27.94) (width 0.5) (layer F.Cu) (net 14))
 (segment (start 129.54 27.94) (end 146.05 27.94) (width 0.5) (layer F.Cu) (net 14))
 (segment (start 147.32 29.21) (end 147.32 30.48) (width 0.5) (layer F.Cu) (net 14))
 (segment (start 146.05 27.94) (end 147.32 29.21) (width 0.5) (layer F.Cu) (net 14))
 (segment (start 114.3 71.12) (end 116.84 68.58) (width 0.5) (layer F.Cu) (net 7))
 (segment (start 116.84 68.58) (end 116.84 54.61) (width 0.5) (layer F.Cu) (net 7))
 (segment (start 139.7 31.75) (end 139.7 30.48) (width 0.5) (layer F.Cu) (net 7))
 (segment (start 116.84 54.61) (end 139.7 31.75) (width 0.5) (layer F.Cu) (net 7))
 (segment (start 137.16 30.48) (end 137.16 29.21) (width 0.5) (layer B.Cu) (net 3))
 (segment (start 137.16 29.21) (end 135.89 27.94) (width 0.5) (layer B.Cu) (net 3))
 (segment (start 135.89 27.94) (end 135.366238 27.94) (width 0.5) (layer B.Cu) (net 3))
 (segment (start 135.366238 27.94) (end 133.35 27.94) (width 0.5) (layer B.Cu) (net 3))
 (segment (start 133.35 27.94) (end 132.08 29.21) (width 0.5) (layer B.Cu) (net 3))
 (segment (start 132.08 29.21) (end 129.54 31.75) (width 0.5) (layer B.Cu) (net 3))
 (segment (start 129.54 31.75) (end 129.54 45.72) (width 0.5) (layer B.Cu) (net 3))
 (segment (start 129.54 45.72) (end 129.54 45.72) (width 0.5) (layer B.Cu) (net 3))
 (via (at 129.54 45.72) (size 0.8) (drill 0.4) (layers F.Cu B.Cu) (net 3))
 (segment (start 129.54 45.72) (end 129.54 45.72) (width 0.5) (layer B.Cu) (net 3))
 (via (at 129.54 45.72) (size 0.8) (drill 0.4) (layers F.Cu B.Cu) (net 3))
 (segment (start 129.54 45.72) (end 129.54 49.53) (width 0.5) (layer F.Cu) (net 3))
 (segment (start 129.54 49.53) (end 119.38 59.69) (width 0.5) (layer F.Cu) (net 3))
 (segment (start 119.38 59.69) (end 119.38 62.23) (width 0.5) (layer F.Cu) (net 3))
 (segment (start 120.65 63.5) (end 121.92 63.5) (width 0.5) (layer F.Cu) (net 3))
 (segment (start 119.38 62.23) (end 120.65 63.5) (width 0.5) (layer F.Cu) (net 3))
 (segment (start 152.4 76.2) (end 152.4 82.8825) (width 1.25) (layer F.Cu) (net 23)))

